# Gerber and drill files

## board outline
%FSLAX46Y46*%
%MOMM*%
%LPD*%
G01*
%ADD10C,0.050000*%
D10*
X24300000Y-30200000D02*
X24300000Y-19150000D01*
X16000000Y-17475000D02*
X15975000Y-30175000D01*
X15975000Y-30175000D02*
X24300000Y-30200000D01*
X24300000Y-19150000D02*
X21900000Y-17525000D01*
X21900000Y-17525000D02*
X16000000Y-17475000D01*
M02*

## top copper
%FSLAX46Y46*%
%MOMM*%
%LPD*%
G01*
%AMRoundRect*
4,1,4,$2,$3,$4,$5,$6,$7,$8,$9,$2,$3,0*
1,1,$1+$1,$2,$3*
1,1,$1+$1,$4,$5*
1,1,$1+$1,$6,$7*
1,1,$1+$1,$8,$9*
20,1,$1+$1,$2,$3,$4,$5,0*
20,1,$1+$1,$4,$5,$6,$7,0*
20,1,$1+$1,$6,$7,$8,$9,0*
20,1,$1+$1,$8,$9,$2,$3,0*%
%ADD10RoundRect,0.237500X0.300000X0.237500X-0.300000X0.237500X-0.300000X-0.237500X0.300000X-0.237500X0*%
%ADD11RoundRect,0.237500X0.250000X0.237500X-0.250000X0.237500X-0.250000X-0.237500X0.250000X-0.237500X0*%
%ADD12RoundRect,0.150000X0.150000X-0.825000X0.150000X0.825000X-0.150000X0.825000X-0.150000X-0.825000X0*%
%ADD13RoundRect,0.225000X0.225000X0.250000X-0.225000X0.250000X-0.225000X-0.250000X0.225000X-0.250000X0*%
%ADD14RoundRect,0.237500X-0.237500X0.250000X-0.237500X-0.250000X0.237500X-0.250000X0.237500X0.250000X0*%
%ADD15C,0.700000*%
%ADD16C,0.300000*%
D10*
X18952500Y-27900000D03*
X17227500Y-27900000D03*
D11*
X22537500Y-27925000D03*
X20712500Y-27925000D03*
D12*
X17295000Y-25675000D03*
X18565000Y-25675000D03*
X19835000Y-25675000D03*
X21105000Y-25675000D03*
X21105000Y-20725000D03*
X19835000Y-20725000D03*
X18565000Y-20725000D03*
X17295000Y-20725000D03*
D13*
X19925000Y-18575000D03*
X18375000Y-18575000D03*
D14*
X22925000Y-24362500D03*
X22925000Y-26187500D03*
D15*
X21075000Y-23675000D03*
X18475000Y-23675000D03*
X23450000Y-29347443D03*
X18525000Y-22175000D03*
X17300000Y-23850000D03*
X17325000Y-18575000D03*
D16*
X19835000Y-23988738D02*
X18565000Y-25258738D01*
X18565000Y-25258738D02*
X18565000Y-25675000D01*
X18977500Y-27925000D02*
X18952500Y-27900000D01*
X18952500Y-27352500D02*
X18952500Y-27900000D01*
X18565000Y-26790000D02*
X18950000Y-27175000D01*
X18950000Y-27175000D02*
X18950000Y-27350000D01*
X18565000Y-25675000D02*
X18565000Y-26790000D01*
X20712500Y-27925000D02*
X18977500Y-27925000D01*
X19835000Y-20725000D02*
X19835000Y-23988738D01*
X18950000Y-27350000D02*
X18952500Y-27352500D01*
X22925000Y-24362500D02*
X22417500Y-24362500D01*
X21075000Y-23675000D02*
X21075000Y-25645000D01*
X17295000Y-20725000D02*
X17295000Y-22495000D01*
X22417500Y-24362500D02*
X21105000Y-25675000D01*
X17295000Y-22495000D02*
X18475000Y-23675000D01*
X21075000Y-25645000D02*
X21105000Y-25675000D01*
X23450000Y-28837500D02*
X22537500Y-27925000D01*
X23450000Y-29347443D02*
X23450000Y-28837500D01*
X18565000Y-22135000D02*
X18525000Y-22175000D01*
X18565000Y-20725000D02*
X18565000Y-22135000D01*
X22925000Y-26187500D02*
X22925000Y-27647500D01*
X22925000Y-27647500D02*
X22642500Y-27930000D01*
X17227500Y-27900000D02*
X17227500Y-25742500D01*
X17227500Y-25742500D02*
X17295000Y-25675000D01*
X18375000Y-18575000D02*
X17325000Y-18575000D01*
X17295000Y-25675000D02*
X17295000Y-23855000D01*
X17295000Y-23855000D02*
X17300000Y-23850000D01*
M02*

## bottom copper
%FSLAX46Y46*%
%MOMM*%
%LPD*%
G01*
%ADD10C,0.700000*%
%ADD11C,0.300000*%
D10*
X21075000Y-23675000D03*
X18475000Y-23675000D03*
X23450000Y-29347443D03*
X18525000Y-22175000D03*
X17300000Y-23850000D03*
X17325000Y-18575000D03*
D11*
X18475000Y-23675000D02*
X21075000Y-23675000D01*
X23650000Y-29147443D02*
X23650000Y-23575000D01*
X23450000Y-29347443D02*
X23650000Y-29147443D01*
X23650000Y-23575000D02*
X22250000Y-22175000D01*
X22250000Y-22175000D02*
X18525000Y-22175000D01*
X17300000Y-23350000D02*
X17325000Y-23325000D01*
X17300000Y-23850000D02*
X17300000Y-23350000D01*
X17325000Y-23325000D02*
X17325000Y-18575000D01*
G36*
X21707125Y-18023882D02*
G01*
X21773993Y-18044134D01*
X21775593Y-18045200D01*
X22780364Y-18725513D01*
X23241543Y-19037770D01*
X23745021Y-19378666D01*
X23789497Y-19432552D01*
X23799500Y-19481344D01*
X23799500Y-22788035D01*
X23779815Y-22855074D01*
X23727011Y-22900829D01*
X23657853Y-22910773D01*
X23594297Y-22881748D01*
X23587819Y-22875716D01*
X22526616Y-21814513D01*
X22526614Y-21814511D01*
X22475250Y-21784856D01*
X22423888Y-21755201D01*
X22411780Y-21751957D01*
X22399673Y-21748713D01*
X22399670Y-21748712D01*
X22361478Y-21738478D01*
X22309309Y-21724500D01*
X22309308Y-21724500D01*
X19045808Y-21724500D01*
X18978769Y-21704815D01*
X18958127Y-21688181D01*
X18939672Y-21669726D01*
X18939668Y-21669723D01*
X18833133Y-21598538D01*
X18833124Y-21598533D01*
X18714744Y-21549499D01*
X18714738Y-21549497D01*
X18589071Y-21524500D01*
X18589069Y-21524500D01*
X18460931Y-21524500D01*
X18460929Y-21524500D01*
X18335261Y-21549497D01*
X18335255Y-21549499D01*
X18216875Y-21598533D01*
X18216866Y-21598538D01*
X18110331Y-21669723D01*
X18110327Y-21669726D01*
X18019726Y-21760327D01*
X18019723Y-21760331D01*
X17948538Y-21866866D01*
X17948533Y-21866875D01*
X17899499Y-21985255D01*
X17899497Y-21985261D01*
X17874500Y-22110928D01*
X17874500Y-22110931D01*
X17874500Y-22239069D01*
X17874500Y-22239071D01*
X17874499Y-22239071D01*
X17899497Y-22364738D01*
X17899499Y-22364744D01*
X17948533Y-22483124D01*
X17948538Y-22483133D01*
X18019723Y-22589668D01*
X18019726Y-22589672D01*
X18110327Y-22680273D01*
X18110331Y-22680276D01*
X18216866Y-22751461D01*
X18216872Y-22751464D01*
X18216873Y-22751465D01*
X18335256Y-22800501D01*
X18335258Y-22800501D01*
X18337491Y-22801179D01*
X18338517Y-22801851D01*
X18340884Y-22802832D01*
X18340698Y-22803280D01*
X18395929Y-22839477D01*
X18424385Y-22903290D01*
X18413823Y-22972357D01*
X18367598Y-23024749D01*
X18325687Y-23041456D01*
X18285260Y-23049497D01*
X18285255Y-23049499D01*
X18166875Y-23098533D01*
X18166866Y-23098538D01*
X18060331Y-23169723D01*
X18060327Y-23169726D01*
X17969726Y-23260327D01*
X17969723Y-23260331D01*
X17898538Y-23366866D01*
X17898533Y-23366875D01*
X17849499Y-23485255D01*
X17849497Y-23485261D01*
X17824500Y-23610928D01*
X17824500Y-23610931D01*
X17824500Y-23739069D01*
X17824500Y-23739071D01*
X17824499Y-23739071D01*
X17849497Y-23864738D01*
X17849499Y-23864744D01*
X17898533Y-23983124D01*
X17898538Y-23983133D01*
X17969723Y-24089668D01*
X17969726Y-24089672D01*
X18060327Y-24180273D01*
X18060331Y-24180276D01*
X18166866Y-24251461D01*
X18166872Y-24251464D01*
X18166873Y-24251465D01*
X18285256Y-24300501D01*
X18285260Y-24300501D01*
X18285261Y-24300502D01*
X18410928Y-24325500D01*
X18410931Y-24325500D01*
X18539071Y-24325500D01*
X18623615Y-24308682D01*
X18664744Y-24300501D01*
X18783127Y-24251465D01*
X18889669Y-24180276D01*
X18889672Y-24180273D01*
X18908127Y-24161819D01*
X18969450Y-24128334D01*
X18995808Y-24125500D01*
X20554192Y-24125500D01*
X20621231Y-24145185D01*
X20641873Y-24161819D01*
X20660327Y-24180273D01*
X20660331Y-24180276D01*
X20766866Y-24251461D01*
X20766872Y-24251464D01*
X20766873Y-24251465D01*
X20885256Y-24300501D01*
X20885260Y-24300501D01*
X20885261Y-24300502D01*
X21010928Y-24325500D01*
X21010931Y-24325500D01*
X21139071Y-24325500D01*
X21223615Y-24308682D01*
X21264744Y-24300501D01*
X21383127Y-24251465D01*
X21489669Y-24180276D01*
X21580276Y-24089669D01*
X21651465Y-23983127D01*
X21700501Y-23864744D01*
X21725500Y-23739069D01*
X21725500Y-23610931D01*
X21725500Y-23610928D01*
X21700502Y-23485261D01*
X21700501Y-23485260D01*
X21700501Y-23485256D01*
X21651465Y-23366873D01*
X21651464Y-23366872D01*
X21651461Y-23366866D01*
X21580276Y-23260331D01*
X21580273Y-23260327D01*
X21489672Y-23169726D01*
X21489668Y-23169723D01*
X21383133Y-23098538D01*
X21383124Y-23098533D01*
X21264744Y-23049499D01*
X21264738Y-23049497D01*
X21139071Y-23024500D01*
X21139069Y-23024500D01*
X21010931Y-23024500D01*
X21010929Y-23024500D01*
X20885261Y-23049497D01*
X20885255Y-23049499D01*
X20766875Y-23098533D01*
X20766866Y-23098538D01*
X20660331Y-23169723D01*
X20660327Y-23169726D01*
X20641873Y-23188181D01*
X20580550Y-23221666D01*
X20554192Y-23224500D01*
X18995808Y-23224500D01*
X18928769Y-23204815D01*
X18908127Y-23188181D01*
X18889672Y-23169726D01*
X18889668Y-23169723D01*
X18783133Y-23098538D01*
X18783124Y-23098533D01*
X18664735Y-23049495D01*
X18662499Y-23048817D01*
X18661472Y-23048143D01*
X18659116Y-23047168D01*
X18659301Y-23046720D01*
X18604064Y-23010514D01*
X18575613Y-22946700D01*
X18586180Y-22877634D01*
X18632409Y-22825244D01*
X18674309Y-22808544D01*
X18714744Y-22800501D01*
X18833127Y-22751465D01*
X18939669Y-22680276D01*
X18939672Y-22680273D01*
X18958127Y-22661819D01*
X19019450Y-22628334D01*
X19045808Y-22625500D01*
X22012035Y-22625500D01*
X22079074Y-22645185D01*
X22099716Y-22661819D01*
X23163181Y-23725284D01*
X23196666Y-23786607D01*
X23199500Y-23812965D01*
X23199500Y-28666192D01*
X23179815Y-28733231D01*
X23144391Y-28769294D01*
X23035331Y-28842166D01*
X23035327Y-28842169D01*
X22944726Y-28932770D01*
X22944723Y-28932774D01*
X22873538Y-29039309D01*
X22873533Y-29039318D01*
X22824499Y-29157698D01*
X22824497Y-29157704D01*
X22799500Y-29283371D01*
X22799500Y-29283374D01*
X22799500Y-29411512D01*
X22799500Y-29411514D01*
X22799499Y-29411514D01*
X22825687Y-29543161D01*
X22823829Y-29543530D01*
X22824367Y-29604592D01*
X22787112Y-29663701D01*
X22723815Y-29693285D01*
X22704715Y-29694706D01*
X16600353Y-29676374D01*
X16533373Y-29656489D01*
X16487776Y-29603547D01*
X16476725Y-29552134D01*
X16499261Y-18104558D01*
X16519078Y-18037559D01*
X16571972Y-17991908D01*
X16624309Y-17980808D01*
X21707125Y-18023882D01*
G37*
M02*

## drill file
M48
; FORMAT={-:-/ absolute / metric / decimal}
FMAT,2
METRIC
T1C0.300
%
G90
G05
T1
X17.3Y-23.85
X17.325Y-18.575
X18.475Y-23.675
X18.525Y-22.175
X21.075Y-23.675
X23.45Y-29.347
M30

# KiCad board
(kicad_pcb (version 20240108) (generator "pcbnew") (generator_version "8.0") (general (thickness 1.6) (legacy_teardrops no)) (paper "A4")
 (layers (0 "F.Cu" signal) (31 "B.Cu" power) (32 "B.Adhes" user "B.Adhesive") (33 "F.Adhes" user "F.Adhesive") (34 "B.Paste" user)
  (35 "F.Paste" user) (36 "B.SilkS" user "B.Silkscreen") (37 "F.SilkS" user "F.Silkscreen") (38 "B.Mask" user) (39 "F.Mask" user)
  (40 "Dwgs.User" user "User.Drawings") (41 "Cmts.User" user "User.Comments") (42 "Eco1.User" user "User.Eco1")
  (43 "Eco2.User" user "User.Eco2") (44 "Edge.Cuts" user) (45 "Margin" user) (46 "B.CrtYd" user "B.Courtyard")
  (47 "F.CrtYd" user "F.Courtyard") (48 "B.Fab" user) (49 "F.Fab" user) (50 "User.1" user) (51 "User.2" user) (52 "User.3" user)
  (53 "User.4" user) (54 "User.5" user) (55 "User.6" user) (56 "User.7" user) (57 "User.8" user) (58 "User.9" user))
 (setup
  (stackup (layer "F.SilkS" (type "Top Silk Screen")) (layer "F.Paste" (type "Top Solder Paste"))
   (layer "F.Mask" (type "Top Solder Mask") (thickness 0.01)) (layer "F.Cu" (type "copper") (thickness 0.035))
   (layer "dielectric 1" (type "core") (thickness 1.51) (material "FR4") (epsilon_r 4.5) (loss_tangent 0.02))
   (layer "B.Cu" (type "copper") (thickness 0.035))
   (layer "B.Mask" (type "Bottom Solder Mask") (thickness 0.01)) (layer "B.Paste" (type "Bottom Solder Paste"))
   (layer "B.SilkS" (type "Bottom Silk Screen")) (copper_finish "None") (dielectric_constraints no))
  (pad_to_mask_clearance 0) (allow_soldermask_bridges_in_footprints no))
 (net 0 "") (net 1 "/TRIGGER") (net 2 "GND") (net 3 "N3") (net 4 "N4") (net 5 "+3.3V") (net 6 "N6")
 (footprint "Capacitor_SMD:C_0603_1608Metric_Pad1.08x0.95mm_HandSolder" (layer "F.Cu") (at 18.09 27.9 180)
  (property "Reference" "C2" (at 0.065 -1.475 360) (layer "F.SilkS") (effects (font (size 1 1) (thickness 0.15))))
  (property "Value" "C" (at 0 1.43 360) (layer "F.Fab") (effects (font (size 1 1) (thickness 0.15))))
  (pad "1" smd roundrect (at -0.8625 0 180) (size 1.075 0.95) (layers "F.Cu" "F.Paste" "F.Mask") (roundrect_rratio 0.25) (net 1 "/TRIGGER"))
  (pad "2" smd roundrect (at 0.8625 0 180) (size 1.075 0.95) (layers "F.Cu" "F.Paste" "F.Mask") (roundrect_rratio 0.25) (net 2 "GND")))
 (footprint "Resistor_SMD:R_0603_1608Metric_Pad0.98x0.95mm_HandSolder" (layer "F.Cu") (at 21.625 27.925 180)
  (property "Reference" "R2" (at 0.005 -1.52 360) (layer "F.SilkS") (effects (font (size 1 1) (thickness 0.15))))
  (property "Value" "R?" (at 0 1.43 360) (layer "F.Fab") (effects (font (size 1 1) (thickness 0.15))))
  (pad "1" smd roundrect (at -0.9125 0 180) (size 0.975 0.95) (layers "F.Cu" "F.Paste" "F.Mask") (roundrect_rratio 0.25) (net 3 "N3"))
  (pad "2" smd roundrect (at 0.9125 0 180) (size 0.975 0.95) (layers "F.Cu" "F.Paste" "F.Mask") (roundrect_rratio 0.25) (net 1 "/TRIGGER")))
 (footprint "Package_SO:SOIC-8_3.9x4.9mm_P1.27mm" (layer "F.Cu") (at 19.2 23.2 90)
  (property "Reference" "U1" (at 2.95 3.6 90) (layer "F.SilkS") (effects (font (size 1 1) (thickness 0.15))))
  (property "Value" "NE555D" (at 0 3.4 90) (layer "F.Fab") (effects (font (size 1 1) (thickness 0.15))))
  (pad "1" smd roundrect (at -2.475 -1.905 90) (size 1.95 0.6) (layers "F.Cu" "F.Paste" "F.Mask") (roundrect_rratio 0.25) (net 2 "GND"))
  (pad "2" smd roundrect (at -2.475 -0.635 90) (size 1.95 0.6) (layers "F.Cu" "F.Paste" "F.Mask") (roundrect_rratio 0.25) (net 1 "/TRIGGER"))
  (pad "3" smd roundrect (at -2.475 0.635 90) (size 1.95 0.6) (layers "F.Cu" "F.Paste" "F.Mask") (roundrect_rratio 0.25) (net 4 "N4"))
  (pad "4" smd roundrect (at -2.475 1.905 90) (size 1.95 0.6) (layers "F.Cu" "F.Paste" "F.Mask") (roundrect_rratio 0.25) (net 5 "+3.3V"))
  (pad "5" smd roundrect (at 2.475 1.905 90) (size 1.95 0.6) (layers "F.Cu" "F.Paste" "F.Mask") (roundrect_rratio 0.25) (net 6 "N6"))
  (pad "6" smd roundrect (at 2.475 0.635 90) (size 1.95 0.6) (layers "F.Cu" "F.Paste" "F.Mask") (roundrect_rratio 0.25) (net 1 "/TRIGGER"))
  (pad "7" smd roundrect (at 2.475 -0.635 90) (size 1.95 0.6) (layers "F.Cu" "F.Paste" "F.Mask") (roundrect_rratio 0.25) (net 3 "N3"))
  (pad "8" smd roundrect (at 2.475 -1.905 90) (size 1.95 0.6) (layers "F.Cu" "F.Paste" "F.Mask") (roundrect_rratio 0.25) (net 5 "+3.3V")))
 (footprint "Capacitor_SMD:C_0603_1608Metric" (layer "F.Cu") (at 19.15 18.575 180)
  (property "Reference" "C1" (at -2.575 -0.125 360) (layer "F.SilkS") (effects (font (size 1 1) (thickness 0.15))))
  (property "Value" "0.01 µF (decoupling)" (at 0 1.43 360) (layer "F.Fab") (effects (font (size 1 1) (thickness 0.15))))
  (pad "1" smd roundrect (at -0.775 0 180) (size 0.9 0.95) (layers "F.Cu" "F.Paste" "F.Mask") (roundrect_rratio 0.25) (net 6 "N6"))
  (pad "2" smd roundrect (at 0.775 0 180) (size 0.9 0.95) (layers "F.Cu" "F.Paste" "F.Mask") (roundrect_rratio 0.25) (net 2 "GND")))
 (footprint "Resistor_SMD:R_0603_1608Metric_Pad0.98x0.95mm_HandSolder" (layer "F.Cu") (at 22.925 25.275 -90)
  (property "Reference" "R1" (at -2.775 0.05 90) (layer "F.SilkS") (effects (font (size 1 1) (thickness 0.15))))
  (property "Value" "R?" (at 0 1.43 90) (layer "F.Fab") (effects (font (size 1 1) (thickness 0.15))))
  (pad "1" smd roundrect (at -0.9125 0 270) (size 0.975 0.95) (layers "F.Cu" "F.Paste" "F.Mask") (roundrect_rratio 0.25) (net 5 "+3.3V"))
  (pad "2" smd roundrect (at 0.9125 0 270) (size 0.975 0.95) (layers "F.Cu" "F.Paste" "F.Mask") (roundrect_rratio 0.25) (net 3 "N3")))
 (gr_line (start 24.3 30.2) (end 24.3 19.15) (stroke (width 0.05) (type default)) (layer "Edge.Cuts"))
 (gr_line (start 16 17.475) (end 15.975 30.175) (stroke (width 0.05) (type default)) (layer "Edge.Cuts"))
 (gr_line (start 15.975 30.175) (end 24.3 30.2) (stroke (width 0.05) (type default)) (layer "Edge.Cuts"))
 (gr_line (start 24.3 19.15) (end 21.9 17.525) (stroke (width 0.05) (type default)) (layer "Edge.Cuts"))
 (gr_line (start 21.9 17.525) (end 16 17.475) (stroke (width 0.05) (type default)) (layer "Edge.Cuts"))
 (segment (start 19.835 23.988738) (end 18.565 25.258738) (width 0.3) (layer "F.Cu") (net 1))
 (segment (start 18.565 25.258738) (end 18.565 25.675) (width 0.3) (layer "F.Cu") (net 1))
 (segment (start 18.9775 27.925) (end 18.9525 27.9) (width 0.3) (layer "F.Cu") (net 1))
 (segment (start 18.9525 27.3525) (end 18.9525 27.9) (width 0.3) (layer "F.Cu") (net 1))
 (segment (start 18.565 26.79) (end 18.95 27.175) (width 0.3) (layer "F.Cu") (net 1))
 (segment (start 18.95 27.175) (end 18.95 27.35) (width 0.3) (layer "F.Cu") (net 1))
 (segment (start 18.565 25.675) (end 18.565 26.79) (width 0.3) (layer "F.Cu") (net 1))
 (segment (start 20.7125 27.925) (end 18.9775 27.925) (width 0.3) (layer "F.Cu") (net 1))
 (segment (start 19.835 20.725) (end 19.835 23.988738) (width 0.3) (layer "F.Cu") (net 1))
 (segment (start 18.95 27.35) (end 18.9525 27.3525) (width 0.3) (layer "F.Cu") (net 1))
 (segment (start 22.925 24.3625) (end 22.4175 24.3625) (width 0.3) (layer "F.Cu") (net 5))
 (segment (start 21.075 23.675) (end 21.075 25.645) (width 0.3) (layer "F.Cu") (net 5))
 (segment (start 17.295 20.725) (end 17.295 22.495) (width 0.3) (layer "F.Cu") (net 5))
 (segment (start 22.4175 24.3625) (end 21.105 25.675) (width 0.3) (layer "F.Cu") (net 5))
 (segment (start 17.295 22.495) (end 18.475 23.675) (width 0.3) (layer "F.Cu") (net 5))
 (segment (start 21.075 25.645) (end 21.105 25.675) (width 0.3) (layer "F.Cu") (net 5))
 (via (at 21.075 23.675) (size 0.7) (drill 0.3) (layers "F.Cu" "B.Cu") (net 5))
 (via (at 18.475 23.675) (size 0.7) (drill 0.3) (layers "F.Cu" "B.Cu") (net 5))
 (segment (start 18.475 23.675) (end 21.075 23.675) (width 0.3) (layer "B.Cu") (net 5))
 (segment (start 23.45 28.8375) (end 22.5375 27.925) (width 0.3) (layer "F.Cu") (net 3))
 (segment (start 23.45 29.347443) (end 23.45 28.8375) (width 0.3) (layer "F.Cu") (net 3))
 (segment (start 18.565 22.135) (end 18.525 22.175) (width 0.3) (layer "F.Cu") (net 3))
 (segment (start 18.565 20.725) (end 18.565 22.135) (width 0.3) (layer "F.Cu") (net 3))
 (segment (start 22.925 26.1875) (end 22.925 27.6475) (width 0.3) (layer "F.Cu") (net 3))
 (segment (start 22.925 27.6475) (end 22.6425 27.93) (width 0.3) (layer "F.Cu") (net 3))
 (via (at 23.45 29.347443) (size 0.7) (drill 0.3) (layers "F.Cu" "B.Cu") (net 3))
 (via (at 18.525 22.175) (size 0.7) (drill 0.3) (layers "F.Cu" "B.Cu") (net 3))
 (segment (start 23.65 29.147443) (end 23.65 23.575) (width 0.3) (layer "B.Cu") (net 3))
 (segment (start 23.45 29.347443) (end 23.65 29.147443) (width 0.3) (layer "B.Cu") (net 3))
 (segment (start 23.65 23.575) (end 22.25 22.175) (width 0.3) (layer "B.Cu") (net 3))
 (segment (start 22.25 22.175) (end 18.525 22.175) (width 0.3) (layer "B.Cu") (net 3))
 (segment (start 17.2275 27.9) (end 17.2275 25.7425) (width 0.3) (layer "F.Cu") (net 2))
 (segment (start 17.2275 25.7425) (end 17.295 25.675) (width 0.3) (layer "F.Cu") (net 2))
 (segment (start 18.375 18.575) (end 17.325 18.575) (width 0.3) (layer "F.Cu") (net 2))
 (segment (start 17.295 25.675) (end 17.295 23.855) (width 0.3) (layer "F.Cu") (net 2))
 (segment (start 17.295 23.855) (end 17.3 23.85) (width 0.3) (layer "F.Cu") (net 2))
 (via (at 17.3 23.85) (size 0.7) (drill 0.3) (layers "F.Cu" "B.Cu") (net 2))
 (via (at 17.325 18.575) (size 0.7) (drill 0.3) (layers "F.Cu" "B.Cu") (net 2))
 (segment (start 17.3 23.35) (end 17.325 23.325) (width 0.3) (layer "B.Cu") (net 2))
 (segment (start 17.3 23.85) (end 17.3 23.35) (width 0.3) (layer "B.Cu") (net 2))
 (segment (start 17.325 23.325) (end 17.325 18.575) (width 0.3) (layer "B.Cu") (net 2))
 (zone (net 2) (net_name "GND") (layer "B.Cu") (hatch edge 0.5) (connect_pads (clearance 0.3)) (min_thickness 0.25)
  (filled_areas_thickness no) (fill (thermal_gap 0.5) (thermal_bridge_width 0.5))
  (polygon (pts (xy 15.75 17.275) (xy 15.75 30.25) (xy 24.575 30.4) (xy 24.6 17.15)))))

